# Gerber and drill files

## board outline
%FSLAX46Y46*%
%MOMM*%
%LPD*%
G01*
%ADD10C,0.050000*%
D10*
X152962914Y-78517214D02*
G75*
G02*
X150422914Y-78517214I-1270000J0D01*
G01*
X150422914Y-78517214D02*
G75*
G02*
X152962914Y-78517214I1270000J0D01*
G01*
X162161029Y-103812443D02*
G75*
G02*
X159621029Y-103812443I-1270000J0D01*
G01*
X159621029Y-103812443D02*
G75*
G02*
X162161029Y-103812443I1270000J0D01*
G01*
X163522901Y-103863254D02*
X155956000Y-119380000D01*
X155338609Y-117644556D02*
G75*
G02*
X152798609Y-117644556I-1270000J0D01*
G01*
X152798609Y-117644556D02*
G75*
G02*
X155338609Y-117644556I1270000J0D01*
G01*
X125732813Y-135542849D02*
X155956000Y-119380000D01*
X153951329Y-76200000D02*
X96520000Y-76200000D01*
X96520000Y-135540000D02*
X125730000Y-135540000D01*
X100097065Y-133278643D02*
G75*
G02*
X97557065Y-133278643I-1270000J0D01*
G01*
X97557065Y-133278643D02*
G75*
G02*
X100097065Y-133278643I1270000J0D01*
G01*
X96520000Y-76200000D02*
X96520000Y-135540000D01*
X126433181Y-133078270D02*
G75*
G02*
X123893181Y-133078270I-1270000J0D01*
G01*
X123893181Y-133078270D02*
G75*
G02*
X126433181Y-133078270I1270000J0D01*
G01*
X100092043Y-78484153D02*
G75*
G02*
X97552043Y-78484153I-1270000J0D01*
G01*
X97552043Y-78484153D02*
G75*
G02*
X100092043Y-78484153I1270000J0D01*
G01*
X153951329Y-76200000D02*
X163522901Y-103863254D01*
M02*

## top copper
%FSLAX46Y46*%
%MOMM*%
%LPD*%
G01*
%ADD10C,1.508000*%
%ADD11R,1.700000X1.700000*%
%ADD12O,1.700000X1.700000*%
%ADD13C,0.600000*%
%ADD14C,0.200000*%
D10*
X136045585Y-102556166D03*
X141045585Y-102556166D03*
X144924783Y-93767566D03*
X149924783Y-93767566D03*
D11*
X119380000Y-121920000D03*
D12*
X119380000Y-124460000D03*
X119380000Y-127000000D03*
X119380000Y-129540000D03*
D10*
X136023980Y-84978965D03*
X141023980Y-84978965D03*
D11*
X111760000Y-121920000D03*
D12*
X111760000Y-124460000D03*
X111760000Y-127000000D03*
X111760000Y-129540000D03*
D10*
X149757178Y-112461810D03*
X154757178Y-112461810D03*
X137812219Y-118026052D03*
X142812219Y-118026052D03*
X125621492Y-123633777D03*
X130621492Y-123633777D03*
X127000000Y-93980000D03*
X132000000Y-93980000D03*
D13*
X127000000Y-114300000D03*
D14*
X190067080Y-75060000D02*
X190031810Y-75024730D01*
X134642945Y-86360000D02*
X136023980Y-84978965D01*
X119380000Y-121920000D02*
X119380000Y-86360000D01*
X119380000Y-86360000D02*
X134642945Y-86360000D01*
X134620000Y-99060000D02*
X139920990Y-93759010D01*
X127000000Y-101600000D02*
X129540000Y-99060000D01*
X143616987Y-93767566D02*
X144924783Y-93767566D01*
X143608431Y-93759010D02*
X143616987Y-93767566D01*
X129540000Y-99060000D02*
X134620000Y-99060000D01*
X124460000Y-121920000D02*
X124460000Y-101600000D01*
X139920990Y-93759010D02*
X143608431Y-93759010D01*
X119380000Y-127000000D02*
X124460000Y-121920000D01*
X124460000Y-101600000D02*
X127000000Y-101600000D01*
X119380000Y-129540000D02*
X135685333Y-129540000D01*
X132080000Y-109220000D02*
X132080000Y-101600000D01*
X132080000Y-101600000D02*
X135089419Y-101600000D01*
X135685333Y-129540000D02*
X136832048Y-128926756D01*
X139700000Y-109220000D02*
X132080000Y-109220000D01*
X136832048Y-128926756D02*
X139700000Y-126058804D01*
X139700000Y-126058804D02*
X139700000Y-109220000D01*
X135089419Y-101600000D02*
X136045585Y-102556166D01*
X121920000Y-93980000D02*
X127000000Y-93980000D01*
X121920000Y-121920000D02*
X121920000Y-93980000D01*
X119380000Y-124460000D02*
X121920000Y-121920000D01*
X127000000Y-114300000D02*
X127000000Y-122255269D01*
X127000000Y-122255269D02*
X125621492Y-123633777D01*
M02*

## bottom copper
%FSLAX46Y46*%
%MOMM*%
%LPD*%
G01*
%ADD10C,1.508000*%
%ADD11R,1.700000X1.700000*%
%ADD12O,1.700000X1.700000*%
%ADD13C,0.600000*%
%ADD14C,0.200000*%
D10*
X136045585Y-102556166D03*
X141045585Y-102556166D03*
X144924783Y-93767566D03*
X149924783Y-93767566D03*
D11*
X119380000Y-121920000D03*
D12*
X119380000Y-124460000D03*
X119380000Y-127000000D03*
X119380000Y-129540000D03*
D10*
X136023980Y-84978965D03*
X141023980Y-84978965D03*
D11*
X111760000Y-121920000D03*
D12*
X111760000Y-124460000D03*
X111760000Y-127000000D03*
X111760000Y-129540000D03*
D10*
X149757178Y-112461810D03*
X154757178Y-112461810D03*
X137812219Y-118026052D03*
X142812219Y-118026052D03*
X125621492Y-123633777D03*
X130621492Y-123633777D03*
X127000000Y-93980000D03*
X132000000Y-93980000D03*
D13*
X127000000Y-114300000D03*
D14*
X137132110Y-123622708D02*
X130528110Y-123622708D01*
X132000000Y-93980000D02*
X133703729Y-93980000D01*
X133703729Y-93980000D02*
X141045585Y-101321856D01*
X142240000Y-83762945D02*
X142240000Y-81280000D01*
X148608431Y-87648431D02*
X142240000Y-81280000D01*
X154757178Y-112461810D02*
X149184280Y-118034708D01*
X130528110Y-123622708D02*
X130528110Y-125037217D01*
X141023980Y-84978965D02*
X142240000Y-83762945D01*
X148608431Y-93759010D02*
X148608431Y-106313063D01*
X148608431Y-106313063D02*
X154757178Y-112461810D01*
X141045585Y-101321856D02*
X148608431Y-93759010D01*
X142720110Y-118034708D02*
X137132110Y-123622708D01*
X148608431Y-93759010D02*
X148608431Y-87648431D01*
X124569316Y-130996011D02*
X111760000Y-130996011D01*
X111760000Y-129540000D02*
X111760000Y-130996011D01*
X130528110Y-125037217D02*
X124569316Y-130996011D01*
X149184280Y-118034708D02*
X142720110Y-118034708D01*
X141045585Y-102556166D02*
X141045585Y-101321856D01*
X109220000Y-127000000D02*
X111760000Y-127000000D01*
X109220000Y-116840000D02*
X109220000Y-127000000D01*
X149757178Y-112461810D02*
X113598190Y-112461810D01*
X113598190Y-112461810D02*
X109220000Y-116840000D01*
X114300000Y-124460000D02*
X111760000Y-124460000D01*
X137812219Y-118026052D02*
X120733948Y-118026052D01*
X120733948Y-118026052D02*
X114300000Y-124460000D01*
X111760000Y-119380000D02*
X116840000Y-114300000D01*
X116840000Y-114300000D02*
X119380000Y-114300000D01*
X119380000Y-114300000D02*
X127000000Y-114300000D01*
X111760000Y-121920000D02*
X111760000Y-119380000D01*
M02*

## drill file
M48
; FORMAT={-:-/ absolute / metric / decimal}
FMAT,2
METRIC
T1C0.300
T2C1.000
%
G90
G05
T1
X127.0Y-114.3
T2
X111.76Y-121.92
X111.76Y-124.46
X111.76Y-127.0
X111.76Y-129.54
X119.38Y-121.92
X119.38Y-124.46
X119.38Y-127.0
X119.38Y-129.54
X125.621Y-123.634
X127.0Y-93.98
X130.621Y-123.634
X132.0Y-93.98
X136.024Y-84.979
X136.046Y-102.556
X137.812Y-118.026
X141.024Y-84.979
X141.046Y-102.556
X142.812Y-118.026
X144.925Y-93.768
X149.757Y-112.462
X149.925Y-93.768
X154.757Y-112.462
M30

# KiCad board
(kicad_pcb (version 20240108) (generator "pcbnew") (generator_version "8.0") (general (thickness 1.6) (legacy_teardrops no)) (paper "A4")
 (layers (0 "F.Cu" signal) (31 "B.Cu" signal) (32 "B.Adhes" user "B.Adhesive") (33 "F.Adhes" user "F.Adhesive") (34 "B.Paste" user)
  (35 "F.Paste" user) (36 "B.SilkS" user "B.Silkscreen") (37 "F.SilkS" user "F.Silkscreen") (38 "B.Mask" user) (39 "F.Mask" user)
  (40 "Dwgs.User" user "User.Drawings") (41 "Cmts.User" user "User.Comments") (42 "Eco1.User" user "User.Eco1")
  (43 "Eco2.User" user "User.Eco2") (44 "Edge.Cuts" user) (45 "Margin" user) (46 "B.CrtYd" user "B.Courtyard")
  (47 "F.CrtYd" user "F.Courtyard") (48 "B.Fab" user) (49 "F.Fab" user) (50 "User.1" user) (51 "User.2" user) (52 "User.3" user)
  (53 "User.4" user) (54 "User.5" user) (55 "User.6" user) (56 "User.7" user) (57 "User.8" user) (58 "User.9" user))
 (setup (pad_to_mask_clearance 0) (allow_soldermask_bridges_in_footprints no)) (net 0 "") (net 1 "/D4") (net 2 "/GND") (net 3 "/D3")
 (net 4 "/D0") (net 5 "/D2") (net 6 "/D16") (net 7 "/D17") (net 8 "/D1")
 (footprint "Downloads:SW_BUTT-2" (layer "F.Cu") (at 138.545585 102.556166)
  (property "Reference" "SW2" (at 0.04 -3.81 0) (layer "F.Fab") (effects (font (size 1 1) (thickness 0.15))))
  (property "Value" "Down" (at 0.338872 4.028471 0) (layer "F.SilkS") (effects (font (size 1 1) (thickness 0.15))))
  (pad "1" thru_hole circle (at -2.5 0) (size 1.508 1.508) (drill 1) (layers "*.Cu" "*.Mask") (remove_unused_layers no) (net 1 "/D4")
   (solder_mask_margin 0.102))
  (pad "2" thru_hole circle (at 2.5 0) (size 1.508 1.508) (drill 1) (layers "*.Cu" "*.Mask") (remove_unused_layers no) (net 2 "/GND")
   (solder_mask_margin 0.102)))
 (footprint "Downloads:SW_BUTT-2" (layer "F.Cu") (at 147.424783 93.767566)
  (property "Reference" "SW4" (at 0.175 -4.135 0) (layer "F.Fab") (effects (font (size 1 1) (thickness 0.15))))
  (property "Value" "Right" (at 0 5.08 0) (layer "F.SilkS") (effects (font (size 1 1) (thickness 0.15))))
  (pad "1" thru_hole circle (at -2.5 0) (size 1.508 1.508) (drill 1) (layers "*.Cu" "*.Mask") (remove_unused_layers no) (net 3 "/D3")
   (solder_mask_margin 0.102))
  (pad "2" thru_hole circle (at 2.5 0) (size 1.508 1.508) (drill 1) (layers "*.Cu" "*.Mask") (remove_unused_layers no) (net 2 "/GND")
   (solder_mask_margin 0.102)))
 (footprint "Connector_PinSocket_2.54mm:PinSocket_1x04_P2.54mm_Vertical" (layer "F.Cu") (at 119.38 121.92)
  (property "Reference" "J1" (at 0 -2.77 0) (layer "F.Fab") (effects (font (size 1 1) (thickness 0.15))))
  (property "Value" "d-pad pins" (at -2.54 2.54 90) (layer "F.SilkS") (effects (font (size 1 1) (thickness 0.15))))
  (pad "1" thru_hole rect (at 0 0) (size 1.7 1.7) (drill 1) (layers "*.Cu" "*.Mask") (remove_unused_layers no) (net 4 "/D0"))
  (pad "2" thru_hole oval (at 0 2.54) (size 1.7 1.7) (drill 1) (layers "*.Cu" "*.Mask") (remove_unused_layers no) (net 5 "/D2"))
  (pad "3" thru_hole oval (at 0 5.08) (size 1.7 1.7) (drill 1) (layers "*.Cu" "*.Mask") (remove_unused_layers no) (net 3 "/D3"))
  (pad "4" thru_hole oval (at 0 7.62) (size 1.7 1.7) (drill 1) (layers "*.Cu" "*.Mask") (remove_unused_layers no) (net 1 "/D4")))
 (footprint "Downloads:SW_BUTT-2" (layer "F.Cu") (at 138.52398 84.978965)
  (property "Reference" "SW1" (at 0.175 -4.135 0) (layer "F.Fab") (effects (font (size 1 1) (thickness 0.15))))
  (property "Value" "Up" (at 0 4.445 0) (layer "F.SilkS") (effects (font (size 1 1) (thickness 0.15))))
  (pad "1" thru_hole circle (at -2.5 0) (size 1.508 1.508) (drill 1) (layers "*.Cu" "*.Mask") (remove_unused_layers no) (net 4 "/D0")
   (solder_mask_margin 0.102))
  (pad "2" thru_hole circle (at 2.5 0) (size 1.508 1.508) (drill 1) (layers "*.Cu" "*.Mask") (remove_unused_layers no) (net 2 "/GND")
   (solder_mask_margin 0.102)))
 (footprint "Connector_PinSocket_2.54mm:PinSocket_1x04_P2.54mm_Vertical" (layer "F.Cu") (at 111.76 121.92)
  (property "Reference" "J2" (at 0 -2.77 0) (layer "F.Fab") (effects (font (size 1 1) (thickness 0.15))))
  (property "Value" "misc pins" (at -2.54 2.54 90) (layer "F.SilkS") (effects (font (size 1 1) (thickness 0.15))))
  (pad "1" thru_hole rect (at 0 0) (size 1.7 1.7) (drill 1) (layers "*.Cu" "*.Mask") (remove_unused_layers no) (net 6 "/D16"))
  (pad "2" thru_hole oval (at 0 2.54) (size 1.7 1.7) (drill 1) (layers "*.Cu" "*.Mask") (remove_unused_layers no) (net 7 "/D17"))
  (pad "3" thru_hole oval (at 0 5.08) (size 1.7 1.7) (drill 1) (layers "*.Cu" "*.Mask") (remove_unused_layers no) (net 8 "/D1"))
  (pad "4" thru_hole oval (at 0 7.62) (size 1.7 1.7) (drill 1) (layers "*.Cu" "*.Mask") (remove_unused_layers no) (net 2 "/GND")))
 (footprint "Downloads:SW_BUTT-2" (layer "F.Cu") (at 152.257178 112.46181)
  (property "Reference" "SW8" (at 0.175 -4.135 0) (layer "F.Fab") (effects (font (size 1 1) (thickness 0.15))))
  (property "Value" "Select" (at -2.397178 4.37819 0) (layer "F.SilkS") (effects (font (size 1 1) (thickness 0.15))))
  (pad "1" thru_hole circle (at -2.5 0) (size 1.508 1.508) (drill 1) (layers "*.Cu" "*.Mask") (remove_unused_layers no) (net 8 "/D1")
   (solder_mask_margin 0.102))
  (pad "2" thru_hole circle (at 2.5 0) (size 1.508 1.508) (drill 1) (layers "*.Cu" "*.Mask") (remove_unused_layers no) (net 2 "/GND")
   (solder_mask_margin 0.102)))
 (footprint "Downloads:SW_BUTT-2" (layer "F.Cu") (at 140.312219 118.026052)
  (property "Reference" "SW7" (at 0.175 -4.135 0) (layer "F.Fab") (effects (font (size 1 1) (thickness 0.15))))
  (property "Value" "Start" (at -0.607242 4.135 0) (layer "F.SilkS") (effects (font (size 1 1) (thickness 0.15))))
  (pad "1" thru_hole circle (at -2.5 0) (size 1.508 1.508) (drill 1) (layers "*.Cu" "*.Mask") (remove_unused_layers no) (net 7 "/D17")
   (solder_mask_margin 0.102))
  (pad "2" thru_hole circle (at 2.5 0) (size 1.508 1.508) (drill 1) (layers "*.Cu" "*.Mask") (remove_unused_layers no) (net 2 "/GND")
   (solder_mask_margin 0.102)))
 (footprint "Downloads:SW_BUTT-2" (layer "F.Cu") (at 128.121492 123.633777)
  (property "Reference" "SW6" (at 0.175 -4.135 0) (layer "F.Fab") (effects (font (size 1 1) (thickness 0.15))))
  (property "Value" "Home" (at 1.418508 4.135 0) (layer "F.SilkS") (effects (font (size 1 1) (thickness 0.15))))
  (pad "1" thru_hole circle (at -2.5 0) (size 1.508 1.508) (drill 1) (layers "*.Cu" "*.Mask") (remove_unused_layers no) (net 6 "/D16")
   (solder_mask_margin 0.102))
  (pad "2" thru_hole circle (at 2.5 0) (size 1.508 1.508) (drill 1) (layers "*.Cu" "*.Mask") (remove_unused_layers no) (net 2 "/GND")
   (solder_mask_margin 0.102)))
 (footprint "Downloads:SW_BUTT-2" (layer "F.Cu") (at 129.5 93.98)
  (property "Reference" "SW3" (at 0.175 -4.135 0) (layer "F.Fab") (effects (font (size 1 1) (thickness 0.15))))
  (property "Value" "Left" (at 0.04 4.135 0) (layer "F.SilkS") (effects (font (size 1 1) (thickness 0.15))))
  (pad "1" thru_hole circle (at -2.5 0) (size 1.508 1.508) (drill 1) (layers "*.Cu" "*.Mask") (remove_unused_layers no) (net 5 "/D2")
   (solder_mask_margin 0.102))
  (pad "2" thru_hole circle (at 2.5 0) (size 1.508 1.508) (drill 1) (layers "*.Cu" "*.Mask") (remove_unused_layers no) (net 2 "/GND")
   (solder_mask_margin 0.102)))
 (gr_circle (center 151.692914 78.517214) (end 150.422914 78.517214) (stroke (width 0.05) (type default)) (fill none) (layer "Edge.Cuts"))
 (gr_circle (center 160.891029 103.812443) (end 162.161029 103.812443) (stroke (width 0.05) (type default)) (fill none) (layer "Edge.Cuts"))
 (gr_line (start 163.522901 103.863254) (end 155.956 119.38) (stroke (width 0.05) (type default)) (layer "Edge.Cuts"))
 (gr_circle (center 154.068609 117.644556) (end 155.338609 117.644556) (stroke (width 0.05) (type default)) (fill none) (layer "Edge.Cuts"))
 (gr_line (start 125.732813 135.542849) (end 155.956 119.38) (stroke (width 0.05) (type default)) (layer "Edge.Cuts"))
 (gr_line (start 153.951329 76.2) (end 96.52 76.2) (stroke (width 0.05) (type default)) (layer "Edge.Cuts"))
 (gr_line (start 96.52 135.54) (end 125.73 135.54) (stroke (width 0.05) (type default)) (layer "Edge.Cuts"))
 (gr_circle (center 98.827065 133.278643) (end 100.097065 133.278643) (stroke (width 0.05) (type default)) (fill none) (layer "Edge.Cuts"))
 (gr_line (start 96.52 76.2) (end 96.52 135.54) (stroke (width 0.05) (type default)) (layer "Edge.Cuts"))
 (gr_circle (center 125.163181 133.07827) (end 126.433181 133.07827) (stroke (width 0.05) (type default)) (fill none) (layer "Edge.Cuts"))
 (gr_circle (center 98.822043 78.484153) (end 98.822043 79.754153) (stroke (width 0.05) (type default)) (fill none) (layer "Edge.Cuts"))
 (gr_line (start 153.951329 76.2) (end 163.522901 103.863254) (stroke (width 0.05) (type default)) (layer "Edge.Cuts"))
 (segment (start 190.06708 75.06) (end 190.03181 75.02473) (width 0.2) (layer "F.Cu") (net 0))
 (segment (start 137.13211 123.622708) (end 130.52811 123.622708) (width 0.2) (layer "B.Cu") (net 2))
 (segment (start 132 93.98) (end 133.703729 93.98) (width 0.2) (layer "B.Cu") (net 2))
 (segment (start 133.703729 93.98) (end 141.045585 101.321856) (width 0.2) (layer "B.Cu") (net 2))
 (segment (start 142.24 83.762945) (end 142.24 81.28) (width 0.2) (layer "B.Cu") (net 2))
 (segment (start 148.608431 87.648431) (end 142.24 81.28) (width 0.2) (layer "B.Cu") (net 2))
 (segment (start 154.757178 112.46181) (end 149.18428 118.034708) (width 0.2) (layer "B.Cu") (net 2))
 (segment (start 130.52811 123.622708) (end 130.52811 125.037217) (width 0.2) (layer "B.Cu") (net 2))
 (segment (start 141.02398 84.978965) (end 142.24 83.762945) (width 0.2) (layer "B.Cu") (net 2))
 (segment (start 148.608431 93.75901) (end 148.608431 106.313063) (width 0.2) (layer "B.Cu") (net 2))
 (segment (start 148.608431 106.313063) (end 154.757178 112.46181) (width 0.2) (layer "B.Cu") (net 2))
 (segment (start 141.045585 101.321856) (end 148.608431 93.75901) (width 0.2) (layer "B.Cu") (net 2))
 (segment (start 142.72011 118.034708) (end 137.13211 123.622708) (width 0.2) (layer "B.Cu") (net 2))
 (segment (start 148.608431 93.75901) (end 148.608431 87.648431) (width 0.2) (layer "B.Cu") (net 2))
 (segment (start 124.569316 130.996011) (end 111.76 130.996011) (width 0.2) (layer "B.Cu") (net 2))
 (segment (start 111.76 129.54) (end 111.76 130.996011) (width 0.2) (layer "B.Cu") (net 2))
 (segment (start 130.52811 125.037217) (end 124.569316 130.996011) (width 0.2) (layer "B.Cu") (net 2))
 (segment (start 149.18428 118.034708) (end 142.72011 118.034708) (width 0.2) (layer "B.Cu") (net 2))
 (segment (start 141.045585 102.556166) (end 141.045585 101.321856) (width 0.2) (layer "B.Cu") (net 2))
 (segment (start 134.642945 86.36) (end 136.02398 84.978965) (width 0.2) (layer "F.Cu") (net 4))
 (segment (start 119.38 121.92) (end 119.38 86.36) (width 0.2) (layer "F.Cu") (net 4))
 (segment (start 119.38 86.36) (end 134.642945 86.36) (width 0.2) (layer "F.Cu") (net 4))
 (segment (start 134.62 99.06) (end 139.92099 93.75901) (width 0.2) (layer "F.Cu") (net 3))
 (segment (start 127 101.6) (end 129.54 99.06) (width 0.2) (layer "F.Cu") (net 3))
 (segment (start 143.616987 93.767566) (end 144.924783 93.767566) (width 0.2) (layer "F.Cu") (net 3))
 (segment (start 143.608431 93.75901) (end 143.616987 93.767566) (width 0.2) (layer "F.Cu") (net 3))
 (segment (start 129.54 99.06) (end 134.62 99.06) (width 0.2) (layer "F.Cu") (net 3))
 (segment (start 124.46 121.92) (end 124.46 101.6) (width 0.2) (layer "F.Cu") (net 3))
 (segment (start 139.92099 93.75901) (end 143.608431 93.75901) (width 0.2) (layer "F.Cu") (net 3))
 (segment (start 119.38 127) (end 124.46 121.92) (width 0.2) (layer "F.Cu") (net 3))
 (segment (start 124.46 101.6) (end 127 101.6) (width 0.2) (layer "F.Cu") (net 3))
 (segment (start 119.38 129.54) (end 135.685333 129.54) (width 0.2) (layer "F.Cu") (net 1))
 (segment (start 132.08 109.22) (end 132.08 101.6) (width 0.2) (layer "F.Cu") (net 1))
 (segment (start 132.08 101.6) (end 135.089419 101.6) (width 0.2) (layer "F.Cu") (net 1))
 (segment (start 135.685333 129.54) (end 136.832048 128.926756) (width 0.2) (layer "F.Cu") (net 1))
 (segment (start 139.7 109.22) (end 132.08 109.22) (width 0.2) (layer "F.Cu") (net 1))
 (segment (start 136.832048 128.926756) (end 139.7 126.058804) (width 0.2) (layer "F.Cu") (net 1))
 (segment (start 139.7 126.058804) (end 139.7 109.22) (width 0.2) (layer "F.Cu") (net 1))
 (segment (start 135.089419 101.6) (end 136.045585 102.556166) (width 0.2) (layer "F.Cu") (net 1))
 (segment (start 121.92 93.98) (end 127 93.98) (width 0.2) (layer "F.Cu") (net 5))
 (segment (start 121.92 121.92) (end 121.92 93.98) (width 0.2) (layer "F.Cu") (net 5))
 (segment (start 119.38 124.46) (end 121.92 121.92) (width 0.2) (layer "F.Cu") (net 5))
 (segment (start 109.22 127) (end 111.76 127) (width 0.2) (layer "B.Cu") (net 8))
 (segment (start 109.22 116.84) (end 109.22 127) (width 0.2) (layer "B.Cu") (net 8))
 (segment (start 149.757178 112.46181) (end 113.59819 112.46181) (width 0.2) (layer "B.Cu") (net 8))
 (segment (start 113.59819 112.46181) (end 109.22 116.84) (width 0.2) (layer "B.Cu") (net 8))
 (segment (start 114.3 124.46) (end 111.76 124.46) (width 0.2) (layer "B.Cu") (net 7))
 (segment (start 137.812219 118.026052) (end 120.733948 118.026052) (width 0.2) (layer "B.Cu") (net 7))
 (segment (start 120.733948 118.026052) (end 114.3 124.46) (width 0.2) (layer "B.Cu") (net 7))
 (segment (start 127 114.3) (end 127 122.255269) (width 0.2) (layer "F.Cu") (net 6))
 (segment (start 127 122.255269) (end 125.621492 123.633777) (width 0.2) (layer "F.Cu") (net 6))
 (via (at 127 114.3) (size 0.6) (drill 0.3) (layers "F.Cu" "B.Cu") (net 6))
 (segment (start 111.76 119.38) (end 116.84 114.3) (width 0.2) (layer "B.Cu") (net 6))
 (segment (start 116.84 114.3) (end 119.38 114.3) (width 0.2) (layer "B.Cu") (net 6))
 (segment (start 119.38 114.3) (end 127 114.3) (width 0.2) (layer "B.Cu") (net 6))
 (segment (start 111.76 121.92) (end 111.76 119.38) (width 0.2) (layer "B.Cu") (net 6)))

